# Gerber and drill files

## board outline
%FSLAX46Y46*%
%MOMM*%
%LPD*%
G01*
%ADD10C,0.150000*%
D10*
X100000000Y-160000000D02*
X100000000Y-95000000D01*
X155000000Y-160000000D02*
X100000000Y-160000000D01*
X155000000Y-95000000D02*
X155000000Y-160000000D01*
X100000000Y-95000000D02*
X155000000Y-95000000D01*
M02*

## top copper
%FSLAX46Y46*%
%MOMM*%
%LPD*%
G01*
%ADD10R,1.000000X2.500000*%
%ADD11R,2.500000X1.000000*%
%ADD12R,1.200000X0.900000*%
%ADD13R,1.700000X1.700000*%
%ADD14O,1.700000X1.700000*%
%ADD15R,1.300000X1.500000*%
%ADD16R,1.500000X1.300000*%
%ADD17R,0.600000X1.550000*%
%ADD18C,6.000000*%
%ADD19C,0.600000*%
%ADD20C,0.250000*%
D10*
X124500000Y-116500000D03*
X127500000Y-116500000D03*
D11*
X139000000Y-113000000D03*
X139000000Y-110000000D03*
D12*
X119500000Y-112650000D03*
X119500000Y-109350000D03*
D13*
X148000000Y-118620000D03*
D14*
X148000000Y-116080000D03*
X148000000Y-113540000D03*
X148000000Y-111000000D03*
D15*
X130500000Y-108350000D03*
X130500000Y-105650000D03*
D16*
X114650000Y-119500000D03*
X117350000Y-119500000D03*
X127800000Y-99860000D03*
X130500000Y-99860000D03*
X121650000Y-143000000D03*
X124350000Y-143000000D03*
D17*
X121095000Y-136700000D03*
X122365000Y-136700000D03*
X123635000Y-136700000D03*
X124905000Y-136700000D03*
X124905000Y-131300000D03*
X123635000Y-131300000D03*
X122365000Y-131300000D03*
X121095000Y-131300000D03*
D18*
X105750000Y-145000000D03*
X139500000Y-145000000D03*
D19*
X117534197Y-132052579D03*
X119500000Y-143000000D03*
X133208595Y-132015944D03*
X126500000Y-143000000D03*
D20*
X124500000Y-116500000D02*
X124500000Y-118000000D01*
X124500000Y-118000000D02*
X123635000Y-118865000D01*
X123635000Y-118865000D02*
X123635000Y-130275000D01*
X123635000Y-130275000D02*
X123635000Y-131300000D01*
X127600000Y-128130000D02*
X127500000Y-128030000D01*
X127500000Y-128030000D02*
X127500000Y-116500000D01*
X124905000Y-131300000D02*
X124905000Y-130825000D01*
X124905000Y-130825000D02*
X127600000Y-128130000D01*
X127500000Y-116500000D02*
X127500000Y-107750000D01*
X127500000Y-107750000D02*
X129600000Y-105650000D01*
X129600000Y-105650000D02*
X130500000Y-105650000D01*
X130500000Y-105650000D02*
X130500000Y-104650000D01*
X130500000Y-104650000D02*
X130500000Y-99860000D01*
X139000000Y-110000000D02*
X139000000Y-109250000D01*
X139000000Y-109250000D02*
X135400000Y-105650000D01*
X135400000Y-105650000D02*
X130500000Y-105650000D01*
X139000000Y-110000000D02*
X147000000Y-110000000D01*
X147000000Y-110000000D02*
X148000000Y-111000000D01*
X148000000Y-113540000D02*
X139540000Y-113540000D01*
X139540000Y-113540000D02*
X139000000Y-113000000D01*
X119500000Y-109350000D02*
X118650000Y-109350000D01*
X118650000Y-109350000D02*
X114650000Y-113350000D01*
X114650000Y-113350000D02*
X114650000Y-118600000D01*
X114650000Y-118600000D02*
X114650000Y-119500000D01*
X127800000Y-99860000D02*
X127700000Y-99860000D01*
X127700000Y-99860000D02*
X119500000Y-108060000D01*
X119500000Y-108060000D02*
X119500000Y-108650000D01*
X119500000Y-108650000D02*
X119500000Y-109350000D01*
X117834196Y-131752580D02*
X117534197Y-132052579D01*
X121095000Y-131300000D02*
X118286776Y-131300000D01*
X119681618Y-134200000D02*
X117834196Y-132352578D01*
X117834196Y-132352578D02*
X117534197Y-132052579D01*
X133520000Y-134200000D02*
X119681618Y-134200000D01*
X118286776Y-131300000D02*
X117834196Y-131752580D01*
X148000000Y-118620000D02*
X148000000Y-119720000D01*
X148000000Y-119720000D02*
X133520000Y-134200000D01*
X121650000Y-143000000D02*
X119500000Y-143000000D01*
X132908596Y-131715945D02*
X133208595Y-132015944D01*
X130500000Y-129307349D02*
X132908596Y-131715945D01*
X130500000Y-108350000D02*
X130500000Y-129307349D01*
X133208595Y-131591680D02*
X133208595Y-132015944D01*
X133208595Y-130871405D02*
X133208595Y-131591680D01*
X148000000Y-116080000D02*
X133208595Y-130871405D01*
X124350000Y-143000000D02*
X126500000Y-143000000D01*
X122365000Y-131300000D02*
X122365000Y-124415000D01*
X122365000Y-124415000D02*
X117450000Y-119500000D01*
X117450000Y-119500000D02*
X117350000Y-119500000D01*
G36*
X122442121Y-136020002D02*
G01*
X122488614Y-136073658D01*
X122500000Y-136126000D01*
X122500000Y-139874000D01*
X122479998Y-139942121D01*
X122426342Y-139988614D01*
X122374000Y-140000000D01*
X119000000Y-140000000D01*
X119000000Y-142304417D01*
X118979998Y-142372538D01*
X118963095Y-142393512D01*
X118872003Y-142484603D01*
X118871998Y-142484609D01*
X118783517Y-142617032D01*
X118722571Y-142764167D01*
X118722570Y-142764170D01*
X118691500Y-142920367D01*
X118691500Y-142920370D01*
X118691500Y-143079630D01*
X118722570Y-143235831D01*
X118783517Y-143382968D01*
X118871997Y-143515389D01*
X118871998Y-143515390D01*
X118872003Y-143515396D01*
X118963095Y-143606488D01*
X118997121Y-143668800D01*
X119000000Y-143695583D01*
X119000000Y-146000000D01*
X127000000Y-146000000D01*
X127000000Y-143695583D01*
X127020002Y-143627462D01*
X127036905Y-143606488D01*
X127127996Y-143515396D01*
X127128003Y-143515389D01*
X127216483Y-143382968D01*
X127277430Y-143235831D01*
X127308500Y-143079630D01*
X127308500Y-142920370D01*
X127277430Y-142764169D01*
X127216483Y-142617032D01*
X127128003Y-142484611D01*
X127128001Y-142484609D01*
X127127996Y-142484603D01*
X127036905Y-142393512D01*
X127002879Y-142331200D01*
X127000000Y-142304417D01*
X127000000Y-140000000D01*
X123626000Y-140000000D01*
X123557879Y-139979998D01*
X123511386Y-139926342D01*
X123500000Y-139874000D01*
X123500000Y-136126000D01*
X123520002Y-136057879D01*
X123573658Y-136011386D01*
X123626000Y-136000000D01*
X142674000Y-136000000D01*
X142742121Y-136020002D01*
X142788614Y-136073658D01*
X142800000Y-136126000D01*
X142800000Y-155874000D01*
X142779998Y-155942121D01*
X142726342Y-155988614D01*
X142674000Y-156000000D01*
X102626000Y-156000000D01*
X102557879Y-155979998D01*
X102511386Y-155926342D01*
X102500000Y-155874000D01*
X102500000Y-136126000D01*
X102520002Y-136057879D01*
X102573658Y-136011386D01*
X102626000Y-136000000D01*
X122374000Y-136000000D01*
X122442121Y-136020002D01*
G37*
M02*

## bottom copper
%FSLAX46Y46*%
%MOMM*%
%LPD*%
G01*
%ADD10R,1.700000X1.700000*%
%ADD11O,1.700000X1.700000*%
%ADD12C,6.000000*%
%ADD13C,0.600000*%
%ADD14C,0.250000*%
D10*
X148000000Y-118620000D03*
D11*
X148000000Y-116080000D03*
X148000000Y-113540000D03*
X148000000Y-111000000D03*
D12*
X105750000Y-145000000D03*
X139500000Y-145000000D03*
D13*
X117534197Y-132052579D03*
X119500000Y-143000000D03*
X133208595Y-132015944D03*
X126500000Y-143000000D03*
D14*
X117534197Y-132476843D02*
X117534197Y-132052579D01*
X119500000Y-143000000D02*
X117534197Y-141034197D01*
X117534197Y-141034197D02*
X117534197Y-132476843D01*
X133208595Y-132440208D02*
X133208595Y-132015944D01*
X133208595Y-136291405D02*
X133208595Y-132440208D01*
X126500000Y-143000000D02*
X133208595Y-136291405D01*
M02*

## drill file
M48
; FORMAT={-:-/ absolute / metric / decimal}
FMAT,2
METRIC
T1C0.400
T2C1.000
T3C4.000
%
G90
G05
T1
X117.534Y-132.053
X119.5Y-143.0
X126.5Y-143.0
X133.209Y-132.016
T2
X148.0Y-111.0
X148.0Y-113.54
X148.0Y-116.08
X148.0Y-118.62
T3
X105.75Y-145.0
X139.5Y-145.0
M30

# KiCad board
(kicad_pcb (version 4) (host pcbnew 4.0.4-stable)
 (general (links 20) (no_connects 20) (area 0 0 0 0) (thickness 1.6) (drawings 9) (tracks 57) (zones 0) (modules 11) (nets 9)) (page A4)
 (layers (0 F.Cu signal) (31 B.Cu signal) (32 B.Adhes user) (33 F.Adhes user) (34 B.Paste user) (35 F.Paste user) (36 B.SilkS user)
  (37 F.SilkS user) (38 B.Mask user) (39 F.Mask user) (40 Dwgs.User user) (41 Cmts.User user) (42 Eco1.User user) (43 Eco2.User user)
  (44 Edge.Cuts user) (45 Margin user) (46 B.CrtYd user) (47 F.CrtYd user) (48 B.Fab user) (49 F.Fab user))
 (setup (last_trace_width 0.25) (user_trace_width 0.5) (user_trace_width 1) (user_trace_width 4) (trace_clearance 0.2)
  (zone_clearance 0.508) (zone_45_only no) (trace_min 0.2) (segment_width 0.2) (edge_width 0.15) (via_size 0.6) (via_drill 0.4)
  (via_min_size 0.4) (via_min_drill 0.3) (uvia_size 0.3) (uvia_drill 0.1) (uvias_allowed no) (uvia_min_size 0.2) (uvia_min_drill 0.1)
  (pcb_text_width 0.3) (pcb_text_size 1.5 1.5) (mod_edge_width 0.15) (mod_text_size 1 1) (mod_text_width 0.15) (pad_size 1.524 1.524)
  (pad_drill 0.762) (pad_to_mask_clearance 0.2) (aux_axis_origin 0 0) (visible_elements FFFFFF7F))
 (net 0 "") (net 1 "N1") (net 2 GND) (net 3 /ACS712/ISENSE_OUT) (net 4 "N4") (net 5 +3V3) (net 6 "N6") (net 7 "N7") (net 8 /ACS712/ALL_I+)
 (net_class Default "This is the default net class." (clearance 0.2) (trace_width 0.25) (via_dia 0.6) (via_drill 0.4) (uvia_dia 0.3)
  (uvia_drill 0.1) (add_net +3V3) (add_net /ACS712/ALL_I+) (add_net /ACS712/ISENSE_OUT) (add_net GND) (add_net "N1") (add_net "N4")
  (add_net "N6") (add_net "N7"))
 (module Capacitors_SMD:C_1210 (layer F.Cu) (at 126 116.5)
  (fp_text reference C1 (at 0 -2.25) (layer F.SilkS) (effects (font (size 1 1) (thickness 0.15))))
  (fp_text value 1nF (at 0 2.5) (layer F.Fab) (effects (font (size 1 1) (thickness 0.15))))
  (pad 1 smd rect (at -1.5 0) (size 1 2.5) (layers F.Cu F.Paste F.Mask) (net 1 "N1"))
  (pad 2 smd rect (at 1.5 0) (size 1 2.5) (layers F.Cu F.Paste F.Mask) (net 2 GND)))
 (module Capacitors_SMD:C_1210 (layer F.Cu) (at 139 111.5 90)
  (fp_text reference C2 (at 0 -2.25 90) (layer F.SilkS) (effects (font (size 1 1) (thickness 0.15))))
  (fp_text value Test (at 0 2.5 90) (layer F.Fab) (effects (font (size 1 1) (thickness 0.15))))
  (pad 1 smd rect (at -1.5 0 90) (size 1 2.5) (layers F.Cu F.Paste F.Mask) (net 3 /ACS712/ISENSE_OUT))
  (pad 2 smd rect (at 1.5 0 90) (size 1 2.5) (layers F.Cu F.Paste F.Mask) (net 2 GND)))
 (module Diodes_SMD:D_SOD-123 (layer F.Cu) (at 119.5 111 90)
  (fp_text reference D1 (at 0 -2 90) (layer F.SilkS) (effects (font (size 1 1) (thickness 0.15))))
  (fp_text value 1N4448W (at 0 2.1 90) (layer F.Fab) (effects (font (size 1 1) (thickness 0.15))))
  (pad 1 smd rect (at -1.65 0 90) (size 0.9 1.2) (layers F.Cu F.Paste F.Mask) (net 3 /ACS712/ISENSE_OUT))
  (pad 2 smd rect (at 1.65 0 90) (size 0.9 1.2) (layers F.Cu F.Paste F.Mask) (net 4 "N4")))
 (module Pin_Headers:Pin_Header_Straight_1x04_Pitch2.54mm (layer B.Cu) (at 148 118.62)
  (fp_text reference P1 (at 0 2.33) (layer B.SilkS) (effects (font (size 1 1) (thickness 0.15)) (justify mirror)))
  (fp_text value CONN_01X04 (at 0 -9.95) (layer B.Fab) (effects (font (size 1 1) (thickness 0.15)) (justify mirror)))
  (pad 1 thru_hole rect (at 0 0) (size 1.7 1.7) (drill 1) (layers *.Cu *.Mask) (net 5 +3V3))
  (pad 2 thru_hole oval (at 0 -2.54) (size 1.7 1.7) (drill 1) (layers *.Cu *.Mask) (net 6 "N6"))
  (pad 3 thru_hole oval (at 0 -5.08) (size 1.7 1.7) (drill 1) (layers *.Cu *.Mask) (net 3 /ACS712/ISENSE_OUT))
  (pad 4 thru_hole oval (at 0 -7.62) (size 1.7 1.7) (drill 1) (layers *.Cu *.Mask) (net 2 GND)))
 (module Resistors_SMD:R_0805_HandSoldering (layer F.Cu) (at 130.5 107 90)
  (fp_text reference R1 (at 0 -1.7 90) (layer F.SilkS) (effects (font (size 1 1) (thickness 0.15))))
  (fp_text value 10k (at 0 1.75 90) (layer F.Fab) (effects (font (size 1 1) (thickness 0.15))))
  (pad 1 smd rect (at -1.35 0 90) (size 1.5 1.3) (layers F.Cu F.Paste F.Mask) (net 6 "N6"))
  (pad 2 smd rect (at 1.35 0 90) (size 1.5 1.3) (layers F.Cu F.Paste F.Mask) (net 2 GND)))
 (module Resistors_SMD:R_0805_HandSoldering (layer F.Cu) (at 116 119.5)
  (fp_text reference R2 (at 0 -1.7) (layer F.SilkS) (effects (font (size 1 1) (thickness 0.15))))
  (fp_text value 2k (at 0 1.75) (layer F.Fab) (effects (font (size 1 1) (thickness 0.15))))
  (pad 1 smd rect (at -1.35 0) (size 1.5 1.3) (layers F.Cu F.Paste F.Mask) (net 4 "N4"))
  (pad 2 smd rect (at 1.35 0) (size 1.5 1.3) (layers F.Cu F.Paste F.Mask) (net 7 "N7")))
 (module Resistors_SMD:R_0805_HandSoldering (layer F.Cu) (at 129.15 99.86)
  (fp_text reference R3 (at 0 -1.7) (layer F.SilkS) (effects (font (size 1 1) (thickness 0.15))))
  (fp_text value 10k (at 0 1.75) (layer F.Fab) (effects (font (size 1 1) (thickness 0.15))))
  (pad 1 smd rect (at -1.35 0) (size 1.5 1.3) (layers F.Cu F.Paste F.Mask) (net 4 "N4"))
  (pad 2 smd rect (at 1.35 0) (size 1.5 1.3) (layers F.Cu F.Paste F.Mask) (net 2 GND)))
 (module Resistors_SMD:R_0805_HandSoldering (layer F.Cu) (at 123 143)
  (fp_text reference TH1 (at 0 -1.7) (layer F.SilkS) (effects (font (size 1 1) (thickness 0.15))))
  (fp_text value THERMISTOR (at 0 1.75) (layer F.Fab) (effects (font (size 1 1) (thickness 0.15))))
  (pad 1 smd rect (at -1.35 0) (size 1.5 1.3) (layers F.Cu F.Paste F.Mask) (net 5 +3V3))
  (pad 2 smd rect (at 1.35 0) (size 1.5 1.3) (layers F.Cu F.Paste F.Mask) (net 6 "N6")))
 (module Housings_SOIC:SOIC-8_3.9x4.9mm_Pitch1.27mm (layer F.Cu) (at 123 134 90)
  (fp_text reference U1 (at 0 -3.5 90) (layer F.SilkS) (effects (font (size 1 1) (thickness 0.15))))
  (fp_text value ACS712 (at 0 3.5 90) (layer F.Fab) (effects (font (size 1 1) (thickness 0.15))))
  (pad 1 smd rect (at -2.7 -1.905 90) (size 1.55 0.6) (layers F.Cu F.Paste F.Mask) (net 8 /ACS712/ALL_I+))
  (pad 2 smd rect (at -2.7 -0.635 90) (size 1.55 0.6) (layers F.Cu F.Paste F.Mask) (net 8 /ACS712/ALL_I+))
  (pad 3 smd rect (at -2.7 0.635 90) (size 1.55 0.6) (layers F.Cu F.Paste F.Mask) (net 8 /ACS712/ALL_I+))
  (pad 4 smd rect (at -2.7 1.905 90) (size 1.55 0.6) (layers F.Cu F.Paste F.Mask) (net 8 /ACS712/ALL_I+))
  (pad 5 smd rect (at 2.7 1.905 90) (size 1.55 0.6) (layers F.Cu F.Paste F.Mask) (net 2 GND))
  (pad 6 smd rect (at 2.7 0.635 90) (size 1.55 0.6) (layers F.Cu F.Paste F.Mask) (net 1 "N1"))
  (pad 7 smd rect (at 2.7 -0.635 90) (size 1.55 0.6) (layers F.Cu F.Paste F.Mask) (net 7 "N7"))
  (pad 8 smd rect (at 2.7 -1.905 90) (size 1.55 0.6) (layers F.Cu F.Paste F.Mask) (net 5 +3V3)))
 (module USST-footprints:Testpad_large (layer F.Cu) (at 105.75 145)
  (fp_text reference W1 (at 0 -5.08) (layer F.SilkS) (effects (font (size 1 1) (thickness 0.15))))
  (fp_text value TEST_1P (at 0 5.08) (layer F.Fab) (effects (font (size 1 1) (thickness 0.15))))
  (pad 1 thru_hole circle (at 0 0) (size 6 6) (drill 4) (layers *.Cu *.Mask) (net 8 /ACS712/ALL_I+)))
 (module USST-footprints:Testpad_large (layer F.Cu) (at 139.5 145)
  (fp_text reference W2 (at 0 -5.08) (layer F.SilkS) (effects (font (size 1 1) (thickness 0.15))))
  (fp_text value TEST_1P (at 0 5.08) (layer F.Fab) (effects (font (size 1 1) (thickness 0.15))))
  (pad 1 thru_hole circle (at 0 0) (size 6 6) (drill 4) (layers *.Cu *.Mask) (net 8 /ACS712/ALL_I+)))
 (gr_line (start 100 160) (end 100 95) (layer Edge.Cuts) (width 0.15))
 (gr_line (start 155 160) (end 100 160) (layer Edge.Cuts) (width 0.15))
 (gr_line (start 155 95) (end 155 160) (layer Edge.Cuts) (width 0.15))
 (gr_line (start 100 95) (end 155 95) (layer Edge.Cuts) (width 0.15))
 (segment (start 124.5 116.5) (end 124.5 118) (width 0.25) (layer F.Cu) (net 1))
 (segment (start 124.5 118) (end 123.635 118.865) (width 0.25) (layer F.Cu) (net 1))
 (segment (start 123.635 118.865) (end 123.635 130.275) (width 0.25) (layer F.Cu) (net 1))
 (segment (start 123.635 130.275) (end 123.635 131.3) (width 0.25) (layer F.Cu) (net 1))
 (segment (start 127.6 128.13) (end 127.5 128.03) (width 0.25) (layer F.Cu) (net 2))
 (segment (start 127.5 128.03) (end 127.5 116.5) (width 0.25) (layer F.Cu) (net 2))
 (segment (start 124.905 131.3) (end 124.905 130.825) (width 0.25) (layer F.Cu) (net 2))
 (segment (start 124.905 130.825) (end 127.6 128.13) (width 0.25) (layer F.Cu) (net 2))
 (segment (start 127.5 116.5) (end 127.5 107.75) (width 0.25) (layer F.Cu) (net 2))
 (segment (start 127.5 107.75) (end 129.6 105.65) (width 0.25) (layer F.Cu) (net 2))
 (segment (start 129.6 105.65) (end 130.5 105.65) (width 0.25) (layer F.Cu) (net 2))
 (segment (start 130.5 105.65) (end 130.5 104.65) (width 0.25) (layer F.Cu) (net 2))
 (segment (start 130.5 104.65) (end 130.5 99.86) (width 0.25) (layer F.Cu) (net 2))
 (segment (start 139 110) (end 139 109.25) (width 0.25) (layer F.Cu) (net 2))
 (segment (start 139 109.25) (end 135.4 105.65) (width 0.25) (layer F.Cu) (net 2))
 (segment (start 135.4 105.65) (end 130.5 105.65) (width 0.25) (layer F.Cu) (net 2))
 (segment (start 139 110) (end 147 110) (width 0.25) (layer F.Cu) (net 2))
 (segment (start 147 110) (end 148 111) (width 0.25) (layer F.Cu) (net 2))
 (segment (start 148 113.54) (end 139.54 113.54) (width 0.25) (layer F.Cu) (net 3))
 (segment (start 139.54 113.54) (end 139 113) (width 0.25) (layer F.Cu) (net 3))
 (segment (start 119.5 109.35) (end 118.65 109.35) (width 0.25) (layer F.Cu) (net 4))
 (segment (start 118.65 109.35) (end 114.65 113.35) (width 0.25) (layer F.Cu) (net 4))
 (segment (start 114.65 113.35) (end 114.65 118.6) (width 0.25) (layer F.Cu) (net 4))
 (segment (start 114.65 118.6) (end 114.65 119.5) (width 0.25) (layer F.Cu) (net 4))
 (segment (start 127.8 99.86) (end 127.7 99.86) (width 0.25) (layer F.Cu) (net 4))
 (segment (start 127.7 99.86) (end 119.5 108.06) (width 0.25) (layer F.Cu) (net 4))
 (segment (start 119.5 108.06) (end 119.5 108.65) (width 0.25) (layer F.Cu) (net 4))
 (segment (start 119.5 108.65) (end 119.5 109.35) (width 0.25) (layer F.Cu) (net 4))
 (segment (start 117.834196 131.75258) (end 117.534197 132.052579) (width 0.25) (layer F.Cu) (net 5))
 (segment (start 121.095 131.3) (end 118.286776 131.3) (width 0.25) (layer F.Cu) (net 5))
 (segment (start 119.681618 134.2) (end 117.834196 132.352578) (width 0.25) (layer F.Cu) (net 5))
 (segment (start 117.834196 132.352578) (end 117.534197 132.052579) (width 0.25) (layer F.Cu) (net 5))
 (segment (start 133.52 134.2) (end 119.681618 134.2) (width 0.25) (layer F.Cu) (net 5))
 (segment (start 118.286776 131.3) (end 117.834196 131.75258) (width 0.25) (layer F.Cu) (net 5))
 (segment (start 148 118.62) (end 148 119.72) (width 0.25) (layer F.Cu) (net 5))
 (segment (start 117.534197 132.476843) (end 117.534197 132.052579) (width 0.25) (layer B.Cu) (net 5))
 (segment (start 119.5 143) (end 117.534197 141.034197) (width 0.25) (layer B.Cu) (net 5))
 (segment (start 117.534197 141.034197) (end 117.534197 132.476843) (width 0.25) (layer B.Cu) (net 5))
 (segment (start 148 119.72) (end 133.52 134.2) (width 0.25) (layer F.Cu) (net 5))
 (via (at 117.534197 132.052579) (size 0.6) (drill 0.4) (layers F.Cu B.Cu) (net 5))
 (segment (start 121.65 143) (end 119.5 143) (width 0.25) (layer F.Cu) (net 5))
 (via (at 119.5 143) (size 0.6) (drill 0.4) (layers F.Cu B.Cu) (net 5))
 (segment (start 132.908596 131.715945) (end 133.208595 132.015944) (width 0.25) (layer F.Cu) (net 6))
 (segment (start 130.5 129.307349) (end 132.908596 131.715945) (width 0.25) (layer F.Cu) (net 6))
 (segment (start 130.5 108.35) (end 130.5 129.307349) (width 0.25) (layer F.Cu) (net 6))
 (segment (start 133.208595 131.59168) (end 133.208595 132.015944) (width 0.25) (layer F.Cu) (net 6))
 (segment (start 133.208595 130.871405) (end 133.208595 131.59168) (width 0.25) (layer F.Cu) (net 6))
 (segment (start 148 116.08) (end 133.208595 130.871405) (width 0.25) (layer F.Cu) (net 6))
 (segment (start 133.208595 132.440208) (end 133.208595 132.015944) (width 0.25) (layer B.Cu) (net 6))
 (segment (start 133.208595 136.291405) (end 133.208595 132.440208) (width 0.25) (layer B.Cu) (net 6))
 (segment (start 126.5 143) (end 133.208595 136.291405) (width 0.25) (layer B.Cu) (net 6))
 (via (at 133.208595 132.015944) (size 0.6) (drill 0.4) (layers F.Cu B.Cu) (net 6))
 (segment (start 124.35 143) (end 126.5 143) (width 0.25) (layer F.Cu) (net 6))
 (via (at 126.5 143) (size 0.6) (drill 0.4) (layers F.Cu B.Cu) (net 6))
 (segment (start 122.365 131.3) (end 122.365 124.415) (width 0.25) (layer F.Cu) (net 7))
 (segment (start 122.365 124.415) (end 117.45 119.5) (width 0.25) (layer F.Cu) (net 7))
 (segment (start 117.45 119.5) (end 117.35 119.5) (width 0.25) (layer F.Cu) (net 7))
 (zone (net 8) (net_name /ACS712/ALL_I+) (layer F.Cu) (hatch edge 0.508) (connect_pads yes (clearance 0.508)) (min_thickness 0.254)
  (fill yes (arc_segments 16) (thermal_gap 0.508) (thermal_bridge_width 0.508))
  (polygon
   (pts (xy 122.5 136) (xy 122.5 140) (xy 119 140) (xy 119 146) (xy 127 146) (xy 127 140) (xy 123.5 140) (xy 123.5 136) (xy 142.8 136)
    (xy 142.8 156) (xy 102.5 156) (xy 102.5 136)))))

